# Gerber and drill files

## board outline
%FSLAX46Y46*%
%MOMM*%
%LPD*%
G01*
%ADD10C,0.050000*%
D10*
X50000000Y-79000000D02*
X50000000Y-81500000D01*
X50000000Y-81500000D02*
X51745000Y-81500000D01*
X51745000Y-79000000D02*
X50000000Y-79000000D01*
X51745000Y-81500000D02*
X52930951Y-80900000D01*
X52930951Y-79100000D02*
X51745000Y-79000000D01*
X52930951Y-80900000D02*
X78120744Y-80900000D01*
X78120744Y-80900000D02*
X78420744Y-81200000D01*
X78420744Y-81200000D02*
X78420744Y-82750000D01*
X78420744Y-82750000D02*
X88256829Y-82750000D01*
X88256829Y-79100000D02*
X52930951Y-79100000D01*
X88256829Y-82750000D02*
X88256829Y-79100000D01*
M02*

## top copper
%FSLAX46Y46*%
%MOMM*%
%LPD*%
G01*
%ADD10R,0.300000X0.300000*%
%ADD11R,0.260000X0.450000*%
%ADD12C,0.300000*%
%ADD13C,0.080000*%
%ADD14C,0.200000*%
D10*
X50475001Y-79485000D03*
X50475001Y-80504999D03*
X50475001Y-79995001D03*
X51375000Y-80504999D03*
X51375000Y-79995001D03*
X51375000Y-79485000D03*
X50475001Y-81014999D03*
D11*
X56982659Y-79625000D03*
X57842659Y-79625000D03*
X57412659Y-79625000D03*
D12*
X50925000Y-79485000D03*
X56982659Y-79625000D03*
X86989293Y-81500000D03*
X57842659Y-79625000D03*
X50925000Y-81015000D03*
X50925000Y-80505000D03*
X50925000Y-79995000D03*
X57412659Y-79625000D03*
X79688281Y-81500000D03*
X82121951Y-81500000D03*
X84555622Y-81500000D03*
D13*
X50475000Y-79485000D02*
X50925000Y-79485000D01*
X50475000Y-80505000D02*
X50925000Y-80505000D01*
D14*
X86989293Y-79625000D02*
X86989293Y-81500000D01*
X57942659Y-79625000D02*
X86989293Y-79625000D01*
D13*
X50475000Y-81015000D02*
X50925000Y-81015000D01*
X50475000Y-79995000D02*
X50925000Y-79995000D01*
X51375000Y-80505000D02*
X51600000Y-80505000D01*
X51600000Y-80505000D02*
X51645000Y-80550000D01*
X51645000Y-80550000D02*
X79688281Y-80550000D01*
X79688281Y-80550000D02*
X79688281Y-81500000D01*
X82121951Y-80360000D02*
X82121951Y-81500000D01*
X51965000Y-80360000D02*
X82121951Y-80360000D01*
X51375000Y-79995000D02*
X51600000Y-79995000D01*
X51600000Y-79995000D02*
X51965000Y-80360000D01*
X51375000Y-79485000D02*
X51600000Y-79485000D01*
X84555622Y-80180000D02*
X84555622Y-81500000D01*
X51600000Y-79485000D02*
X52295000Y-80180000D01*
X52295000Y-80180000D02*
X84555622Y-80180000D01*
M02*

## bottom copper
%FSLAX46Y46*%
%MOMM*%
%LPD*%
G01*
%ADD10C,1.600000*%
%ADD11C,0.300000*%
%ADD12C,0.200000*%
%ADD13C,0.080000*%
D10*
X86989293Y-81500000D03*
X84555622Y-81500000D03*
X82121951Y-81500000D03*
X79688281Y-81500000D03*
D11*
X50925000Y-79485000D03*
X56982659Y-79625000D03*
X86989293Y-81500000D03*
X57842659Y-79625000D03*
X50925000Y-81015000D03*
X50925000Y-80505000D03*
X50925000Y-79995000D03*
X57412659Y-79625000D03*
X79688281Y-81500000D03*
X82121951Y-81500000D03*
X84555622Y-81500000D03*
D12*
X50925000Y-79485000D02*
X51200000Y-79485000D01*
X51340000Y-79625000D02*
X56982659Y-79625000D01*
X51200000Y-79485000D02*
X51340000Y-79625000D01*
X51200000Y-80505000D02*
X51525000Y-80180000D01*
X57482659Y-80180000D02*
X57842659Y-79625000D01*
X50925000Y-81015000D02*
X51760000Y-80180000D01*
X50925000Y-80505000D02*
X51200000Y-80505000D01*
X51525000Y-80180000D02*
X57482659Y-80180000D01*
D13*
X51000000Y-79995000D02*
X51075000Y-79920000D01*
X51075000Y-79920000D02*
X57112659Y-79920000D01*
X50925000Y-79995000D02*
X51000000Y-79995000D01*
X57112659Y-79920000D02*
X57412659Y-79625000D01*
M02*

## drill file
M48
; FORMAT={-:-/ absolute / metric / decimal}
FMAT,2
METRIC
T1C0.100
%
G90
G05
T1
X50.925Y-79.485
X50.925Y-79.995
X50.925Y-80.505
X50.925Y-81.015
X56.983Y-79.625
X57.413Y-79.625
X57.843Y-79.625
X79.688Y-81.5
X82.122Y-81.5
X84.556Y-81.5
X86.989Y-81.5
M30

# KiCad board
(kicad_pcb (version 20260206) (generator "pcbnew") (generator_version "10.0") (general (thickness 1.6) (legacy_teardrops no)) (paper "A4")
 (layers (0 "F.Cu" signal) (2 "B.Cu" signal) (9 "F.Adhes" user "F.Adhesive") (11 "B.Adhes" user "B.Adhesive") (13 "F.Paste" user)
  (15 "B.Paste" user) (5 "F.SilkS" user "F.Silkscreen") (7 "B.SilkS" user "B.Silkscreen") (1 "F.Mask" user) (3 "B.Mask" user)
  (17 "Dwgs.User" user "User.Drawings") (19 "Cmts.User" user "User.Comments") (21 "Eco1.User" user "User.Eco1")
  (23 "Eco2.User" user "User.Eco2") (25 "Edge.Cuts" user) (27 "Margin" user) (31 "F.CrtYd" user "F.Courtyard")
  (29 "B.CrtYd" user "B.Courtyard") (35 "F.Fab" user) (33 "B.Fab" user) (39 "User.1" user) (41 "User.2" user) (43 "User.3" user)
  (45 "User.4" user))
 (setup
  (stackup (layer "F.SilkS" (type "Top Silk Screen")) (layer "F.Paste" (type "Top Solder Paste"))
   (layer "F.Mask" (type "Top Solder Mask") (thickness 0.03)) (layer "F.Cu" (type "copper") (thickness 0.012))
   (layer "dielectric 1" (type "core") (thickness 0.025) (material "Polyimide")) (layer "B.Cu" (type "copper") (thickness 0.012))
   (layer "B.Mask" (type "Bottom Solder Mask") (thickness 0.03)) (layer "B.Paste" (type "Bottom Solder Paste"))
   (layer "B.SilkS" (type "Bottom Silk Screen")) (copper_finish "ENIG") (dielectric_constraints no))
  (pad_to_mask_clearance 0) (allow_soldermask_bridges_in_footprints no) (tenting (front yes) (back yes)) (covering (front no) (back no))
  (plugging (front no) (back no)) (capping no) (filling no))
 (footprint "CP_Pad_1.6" (layer "F.Cu") (at 82.121951 81.5)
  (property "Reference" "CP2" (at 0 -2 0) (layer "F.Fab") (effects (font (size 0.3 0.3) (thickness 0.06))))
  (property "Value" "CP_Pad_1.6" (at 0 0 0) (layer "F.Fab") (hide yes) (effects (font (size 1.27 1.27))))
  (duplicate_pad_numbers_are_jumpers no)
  (pad "1" smd circle (at 0 0) (size 1.6 1.6) (layers "B.Cu" "B.Mask") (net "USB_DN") (solder_mask_margin 0.1)))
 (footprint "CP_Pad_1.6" (layer "F.Cu") (at 86.989293 81.5)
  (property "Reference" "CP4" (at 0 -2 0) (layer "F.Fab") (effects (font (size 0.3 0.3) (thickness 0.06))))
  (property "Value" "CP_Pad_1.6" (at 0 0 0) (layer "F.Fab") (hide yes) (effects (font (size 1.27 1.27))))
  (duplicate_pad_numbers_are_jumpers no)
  (pad "1" smd circle (at 0 0) (size 1.6 1.6) (layers "B.Cu" "B.Mask") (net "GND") (solder_mask_margin 0.1)))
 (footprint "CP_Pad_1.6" (layer "F.Cu") (at 84.555622 81.5)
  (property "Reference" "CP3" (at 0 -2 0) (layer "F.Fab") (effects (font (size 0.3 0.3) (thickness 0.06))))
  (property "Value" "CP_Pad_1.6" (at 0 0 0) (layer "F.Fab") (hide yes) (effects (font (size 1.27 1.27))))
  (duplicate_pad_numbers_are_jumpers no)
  (pad "1" smd circle (at 0 0) (size 1.6 1.6) (layers "B.Cu" "B.Mask") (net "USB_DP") (solder_mask_margin 0.1)))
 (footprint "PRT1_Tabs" (layer "F.Cu") (at 57.412659 79.625)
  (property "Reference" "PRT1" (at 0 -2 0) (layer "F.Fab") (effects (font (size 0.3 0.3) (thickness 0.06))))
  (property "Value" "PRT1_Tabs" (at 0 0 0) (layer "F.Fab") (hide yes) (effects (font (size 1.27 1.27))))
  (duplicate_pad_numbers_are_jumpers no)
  (pad "1" smd rect (at -0.43 0) (size 0.26 0.45) (layers "F.Cu" "F.Mask") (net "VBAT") (solder_mask_margin 0.05) (thermal_bridge_angle 45))
  (pad "2" smd rect (at 0.43 0) (size 0.26 0.45) (layers "F.Cu" "F.Mask") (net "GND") (solder_mask_margin 0.05) (thermal_bridge_angle 45))
  (pad "3" smd rect (at 0 0) (size 0.26 0.45) (layers "F.Cu" "F.Mask") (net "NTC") (solder_mask_margin 0.05) (thermal_bridge_angle 45)))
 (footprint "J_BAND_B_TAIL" (layer "F.Cu") (at 50.9 80.25)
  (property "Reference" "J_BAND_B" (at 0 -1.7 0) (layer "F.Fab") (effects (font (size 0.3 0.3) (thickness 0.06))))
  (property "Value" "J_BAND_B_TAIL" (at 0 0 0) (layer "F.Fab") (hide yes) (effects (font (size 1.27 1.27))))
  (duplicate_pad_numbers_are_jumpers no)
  (pad "1" smd rect (at -0.424999 -0.765) (size 0.3 0.3) (layers "F.Cu" "F.Mask") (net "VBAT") (solder_mask_margin 0.05)
   (thermal_bridge_angle 45))
  (pad "2" smd rect (at -0.424999 0.254999) (size 0.3 0.3) (layers "F.Cu" "F.Mask") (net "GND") (solder_mask_margin 0.05)
   (thermal_bridge_angle 45))
  (pad "3" smd rect (at -0.424999 -0.254999) (size 0.3 0.3) (layers "F.Cu" "F.Mask") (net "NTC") (solder_mask_margin 0.05)
   (thermal_bridge_angle 45))
  (pad "4" smd rect (at 0.475 0.254999) (size 0.3 0.3) (layers "F.Cu" "F.Mask") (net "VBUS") (solder_mask_margin 0.05)
   (thermal_bridge_angle 45))
  (pad "5" smd rect (at 0.475 -0.254999) (size 0.3 0.3) (layers "F.Cu" "F.Mask") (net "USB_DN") (solder_mask_margin 0.05)
   (thermal_bridge_angle 45))
  (pad "6" smd rect (at 0.475 -0.765) (size 0.3 0.3) (layers "F.Cu" "F.Mask") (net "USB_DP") (solder_mask_margin 0.05)
   (thermal_bridge_angle 45))
  (pad "7" smd rect (at -0.424999 0.764999) (size 0.3 0.3) (layers "F.Cu" "F.Mask") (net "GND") (solder_mask_margin 0.05)
   (thermal_bridge_angle 45)))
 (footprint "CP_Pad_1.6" (layer "F.Cu") (at 79.688281 81.5)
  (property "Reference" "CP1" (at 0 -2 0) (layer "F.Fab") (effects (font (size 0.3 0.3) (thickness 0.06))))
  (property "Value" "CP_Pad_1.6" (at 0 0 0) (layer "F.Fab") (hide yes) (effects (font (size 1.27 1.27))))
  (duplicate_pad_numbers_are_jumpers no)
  (pad "1" smd circle (at 0 0) (size 1.6 1.6) (layers "B.Cu" "B.Mask") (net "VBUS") (solder_mask_margin 0.1)))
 (gr_line (start 50 79) (end 50 81.5) (stroke (width 0.05) (type default)) (layer "Edge.Cuts"))
 (gr_line (start 50 81.5) (end 51.745 81.5) (stroke (width 0.05) (type default)) (layer "Edge.Cuts"))
 (gr_line (start 51.745 79) (end 50 79) (stroke (width 0.05) (type default)) (layer "Edge.Cuts"))
 (gr_line (start 51.745 81.5) (end 52.930951 80.9) (stroke (width 0.05) (type default)) (layer "Edge.Cuts"))
 (gr_line (start 52.930951 79.1) (end 51.745 79) (stroke (width 0.05) (type default)) (layer "Edge.Cuts"))
 (gr_line (start 52.930951 80.9) (end 78.120744 80.9) (stroke (width 0.05) (type default)) (layer "Edge.Cuts"))
 (gr_line (start 78.120744 80.9) (end 78.420744 81.2) (stroke (width 0.05) (type default)) (layer "Edge.Cuts"))
 (gr_line (start 78.420744 81.2) (end 78.420744 82.75) (stroke (width 0.05) (type default)) (layer "Edge.Cuts"))
 (gr_line (start 78.420744 82.75) (end 88.256829 82.75) (stroke (width 0.05) (type default)) (layer "Edge.Cuts"))
 (gr_line (start 88.256829 79.1) (end 52.930951 79.1) (stroke (width 0.05) (type default)) (layer "Edge.Cuts"))
 (gr_line (start 88.256829 82.75) (end 88.256829 79.1) (stroke (width 0.05) (type default)) (layer "Edge.Cuts"))
 (segment (start 50.475 79.485) (end 50.925 79.485) (width 0.08) (layer "F.Cu") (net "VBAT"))
 (via (at 56.982659 79.625) (size 0.3) (drill 0.1) (layers "F.Cu" "B.Cu") (tenting (front yes) (back yes)) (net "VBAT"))
 (via (at 50.925 79.485) (size 0.3) (drill 0.1) (layers "F.Cu" "B.Cu") (tenting (front yes) (back yes)) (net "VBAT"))
 (segment (start 51.2 79.485) (end 51.34 79.625) (width 0.2) (layer "B.Cu") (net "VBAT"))
 (segment (start 50.925 79.485) (end 51.2 79.485) (width 0.2) (layer "B.Cu") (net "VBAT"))
 (segment (start 51.34 79.625) (end 56.982659 79.625) (width 0.2) (layer "B.Cu") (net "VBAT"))
 (segment (start 50.475 80.505) (end 50.925 80.505) (width 0.08) (layer "F.Cu") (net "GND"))
 (segment (start 57.942659 79.625) (end 86.989293 79.625) (width 0.2) (layer "F.Cu") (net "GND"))
 (segment (start 50.475 81.015) (end 50.925 81.015) (width 0.08) (layer "F.Cu") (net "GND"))
 (segment (start 86.989293 79.625) (end 86.989293 81.5) (width 0.2) (layer "F.Cu") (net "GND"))
 (via (at 57.842659 79.625) (size 0.3) (drill 0.1) (layers "F.Cu" "B.Cu") (tenting (front yes) (back yes)) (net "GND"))
 (via (at 50.925 80.505) (size 0.3) (drill 0.1) (layers "F.Cu" "B.Cu") (tenting (front yes) (back yes)) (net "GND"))
 (via (at 86.989293 81.5) (size 0.3) (drill 0.1) (layers "F.Cu" "B.Cu") (tenting (front yes) (back yes)) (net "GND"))
 (via (at 50.925 81.015) (size 0.3) (drill 0.1) (layers "F.Cu" "B.Cu") (tenting (front yes) (back yes)) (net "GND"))
 (segment (start 51.525 80.18) (end 57.482659 80.18) (width 0.2) (layer "B.Cu") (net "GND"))
 (segment (start 50.925 81.015) (end 51.76 80.18) (width 0.2) (layer "B.Cu") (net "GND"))
 (segment (start 51.2 80.505) (end 51.525 80.18) (width 0.2) (layer "B.Cu") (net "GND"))
 (segment (start 57.482659 80.18) (end 57.842659 79.625) (width 0.2) (layer "B.Cu") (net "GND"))
 (segment (start 50.925 80.505) (end 51.2 80.505) (width 0.2) (layer "B.Cu") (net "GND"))
 (segment (start 50.475 79.995) (end 50.925 79.995) (width 0.08) (layer "F.Cu") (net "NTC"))
 (via (at 57.412659 79.625) (size 0.3) (drill 0.1) (layers "F.Cu" "B.Cu") (tenting (front yes) (back yes)) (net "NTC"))
 (via (at 50.925 79.995) (size 0.3) (drill 0.1) (layers "F.Cu" "B.Cu") (tenting (front yes) (back yes)) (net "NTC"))
 (segment (start 51 79.995) (end 51.075 79.92) (width 0.08) (layer "B.Cu") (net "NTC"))
 (segment (start 51.075 79.92) (end 57.112659 79.92) (width 0.08) (layer "B.Cu") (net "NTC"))
 (segment (start 50.925 79.995) (end 51 79.995) (width 0.08) (layer "B.Cu") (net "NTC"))
 (segment (start 57.112659 79.92) (end 57.412659 79.625) (width 0.08) (layer "B.Cu") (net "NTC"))
 (segment (start 51.375 80.505) (end 51.6 80.505) (width 0.08) (layer "F.Cu") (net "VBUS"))
 (segment (start 51.6 80.505) (end 51.645 80.55) (width 0.08) (layer "F.Cu") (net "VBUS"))
 (segment (start 79.688281 80.55) (end 79.688281 81.5) (width 0.08) (layer "F.Cu") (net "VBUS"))
 (segment (start 51.645 80.55) (end 79.688281 80.55) (width 0.08) (layer "F.Cu") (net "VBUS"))
 (via (at 79.688281 81.5) (size 0.3) (drill 0.1) (layers "F.Cu" "B.Cu") (tenting (front yes) (back yes)) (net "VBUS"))
 (segment (start 82.121951 80.36) (end 82.121951 81.5) (width 0.08) (layer "F.Cu") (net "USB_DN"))
 (segment (start 51.6 79.995) (end 51.965 80.36) (width 0.08) (layer "F.Cu") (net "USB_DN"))
 (segment (start 51.965 80.36) (end 82.121951 80.36) (width 0.08) (layer "F.Cu") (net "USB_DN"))
 (segment (start 51.375 79.995) (end 51.6 79.995) (width 0.08) (layer "F.Cu") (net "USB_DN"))
 (via (at 82.121951 81.5) (size 0.3) (drill 0.1) (layers "F.Cu" "B.Cu") (tenting (front yes) (back yes)) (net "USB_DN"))
 (segment (start 51.375 79.485) (end 51.6 79.485) (width 0.08) (layer "F.Cu") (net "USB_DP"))
 (segment (start 52.295 80.18) (end 84.555622 80.18) (width 0.08) (layer "F.Cu") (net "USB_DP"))
 (segment (start 84.555622 80.18) (end 84.555622 81.5) (width 0.08) (layer "F.Cu") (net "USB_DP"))
 (segment (start 51.6 79.485) (end 52.295 80.18) (width 0.08) (layer "F.Cu") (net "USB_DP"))
 (via (at 84.555622 81.5) (size 0.3) (drill 0.1) (layers "F.Cu" "B.Cu") (tenting (front yes) (back yes)) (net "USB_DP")))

